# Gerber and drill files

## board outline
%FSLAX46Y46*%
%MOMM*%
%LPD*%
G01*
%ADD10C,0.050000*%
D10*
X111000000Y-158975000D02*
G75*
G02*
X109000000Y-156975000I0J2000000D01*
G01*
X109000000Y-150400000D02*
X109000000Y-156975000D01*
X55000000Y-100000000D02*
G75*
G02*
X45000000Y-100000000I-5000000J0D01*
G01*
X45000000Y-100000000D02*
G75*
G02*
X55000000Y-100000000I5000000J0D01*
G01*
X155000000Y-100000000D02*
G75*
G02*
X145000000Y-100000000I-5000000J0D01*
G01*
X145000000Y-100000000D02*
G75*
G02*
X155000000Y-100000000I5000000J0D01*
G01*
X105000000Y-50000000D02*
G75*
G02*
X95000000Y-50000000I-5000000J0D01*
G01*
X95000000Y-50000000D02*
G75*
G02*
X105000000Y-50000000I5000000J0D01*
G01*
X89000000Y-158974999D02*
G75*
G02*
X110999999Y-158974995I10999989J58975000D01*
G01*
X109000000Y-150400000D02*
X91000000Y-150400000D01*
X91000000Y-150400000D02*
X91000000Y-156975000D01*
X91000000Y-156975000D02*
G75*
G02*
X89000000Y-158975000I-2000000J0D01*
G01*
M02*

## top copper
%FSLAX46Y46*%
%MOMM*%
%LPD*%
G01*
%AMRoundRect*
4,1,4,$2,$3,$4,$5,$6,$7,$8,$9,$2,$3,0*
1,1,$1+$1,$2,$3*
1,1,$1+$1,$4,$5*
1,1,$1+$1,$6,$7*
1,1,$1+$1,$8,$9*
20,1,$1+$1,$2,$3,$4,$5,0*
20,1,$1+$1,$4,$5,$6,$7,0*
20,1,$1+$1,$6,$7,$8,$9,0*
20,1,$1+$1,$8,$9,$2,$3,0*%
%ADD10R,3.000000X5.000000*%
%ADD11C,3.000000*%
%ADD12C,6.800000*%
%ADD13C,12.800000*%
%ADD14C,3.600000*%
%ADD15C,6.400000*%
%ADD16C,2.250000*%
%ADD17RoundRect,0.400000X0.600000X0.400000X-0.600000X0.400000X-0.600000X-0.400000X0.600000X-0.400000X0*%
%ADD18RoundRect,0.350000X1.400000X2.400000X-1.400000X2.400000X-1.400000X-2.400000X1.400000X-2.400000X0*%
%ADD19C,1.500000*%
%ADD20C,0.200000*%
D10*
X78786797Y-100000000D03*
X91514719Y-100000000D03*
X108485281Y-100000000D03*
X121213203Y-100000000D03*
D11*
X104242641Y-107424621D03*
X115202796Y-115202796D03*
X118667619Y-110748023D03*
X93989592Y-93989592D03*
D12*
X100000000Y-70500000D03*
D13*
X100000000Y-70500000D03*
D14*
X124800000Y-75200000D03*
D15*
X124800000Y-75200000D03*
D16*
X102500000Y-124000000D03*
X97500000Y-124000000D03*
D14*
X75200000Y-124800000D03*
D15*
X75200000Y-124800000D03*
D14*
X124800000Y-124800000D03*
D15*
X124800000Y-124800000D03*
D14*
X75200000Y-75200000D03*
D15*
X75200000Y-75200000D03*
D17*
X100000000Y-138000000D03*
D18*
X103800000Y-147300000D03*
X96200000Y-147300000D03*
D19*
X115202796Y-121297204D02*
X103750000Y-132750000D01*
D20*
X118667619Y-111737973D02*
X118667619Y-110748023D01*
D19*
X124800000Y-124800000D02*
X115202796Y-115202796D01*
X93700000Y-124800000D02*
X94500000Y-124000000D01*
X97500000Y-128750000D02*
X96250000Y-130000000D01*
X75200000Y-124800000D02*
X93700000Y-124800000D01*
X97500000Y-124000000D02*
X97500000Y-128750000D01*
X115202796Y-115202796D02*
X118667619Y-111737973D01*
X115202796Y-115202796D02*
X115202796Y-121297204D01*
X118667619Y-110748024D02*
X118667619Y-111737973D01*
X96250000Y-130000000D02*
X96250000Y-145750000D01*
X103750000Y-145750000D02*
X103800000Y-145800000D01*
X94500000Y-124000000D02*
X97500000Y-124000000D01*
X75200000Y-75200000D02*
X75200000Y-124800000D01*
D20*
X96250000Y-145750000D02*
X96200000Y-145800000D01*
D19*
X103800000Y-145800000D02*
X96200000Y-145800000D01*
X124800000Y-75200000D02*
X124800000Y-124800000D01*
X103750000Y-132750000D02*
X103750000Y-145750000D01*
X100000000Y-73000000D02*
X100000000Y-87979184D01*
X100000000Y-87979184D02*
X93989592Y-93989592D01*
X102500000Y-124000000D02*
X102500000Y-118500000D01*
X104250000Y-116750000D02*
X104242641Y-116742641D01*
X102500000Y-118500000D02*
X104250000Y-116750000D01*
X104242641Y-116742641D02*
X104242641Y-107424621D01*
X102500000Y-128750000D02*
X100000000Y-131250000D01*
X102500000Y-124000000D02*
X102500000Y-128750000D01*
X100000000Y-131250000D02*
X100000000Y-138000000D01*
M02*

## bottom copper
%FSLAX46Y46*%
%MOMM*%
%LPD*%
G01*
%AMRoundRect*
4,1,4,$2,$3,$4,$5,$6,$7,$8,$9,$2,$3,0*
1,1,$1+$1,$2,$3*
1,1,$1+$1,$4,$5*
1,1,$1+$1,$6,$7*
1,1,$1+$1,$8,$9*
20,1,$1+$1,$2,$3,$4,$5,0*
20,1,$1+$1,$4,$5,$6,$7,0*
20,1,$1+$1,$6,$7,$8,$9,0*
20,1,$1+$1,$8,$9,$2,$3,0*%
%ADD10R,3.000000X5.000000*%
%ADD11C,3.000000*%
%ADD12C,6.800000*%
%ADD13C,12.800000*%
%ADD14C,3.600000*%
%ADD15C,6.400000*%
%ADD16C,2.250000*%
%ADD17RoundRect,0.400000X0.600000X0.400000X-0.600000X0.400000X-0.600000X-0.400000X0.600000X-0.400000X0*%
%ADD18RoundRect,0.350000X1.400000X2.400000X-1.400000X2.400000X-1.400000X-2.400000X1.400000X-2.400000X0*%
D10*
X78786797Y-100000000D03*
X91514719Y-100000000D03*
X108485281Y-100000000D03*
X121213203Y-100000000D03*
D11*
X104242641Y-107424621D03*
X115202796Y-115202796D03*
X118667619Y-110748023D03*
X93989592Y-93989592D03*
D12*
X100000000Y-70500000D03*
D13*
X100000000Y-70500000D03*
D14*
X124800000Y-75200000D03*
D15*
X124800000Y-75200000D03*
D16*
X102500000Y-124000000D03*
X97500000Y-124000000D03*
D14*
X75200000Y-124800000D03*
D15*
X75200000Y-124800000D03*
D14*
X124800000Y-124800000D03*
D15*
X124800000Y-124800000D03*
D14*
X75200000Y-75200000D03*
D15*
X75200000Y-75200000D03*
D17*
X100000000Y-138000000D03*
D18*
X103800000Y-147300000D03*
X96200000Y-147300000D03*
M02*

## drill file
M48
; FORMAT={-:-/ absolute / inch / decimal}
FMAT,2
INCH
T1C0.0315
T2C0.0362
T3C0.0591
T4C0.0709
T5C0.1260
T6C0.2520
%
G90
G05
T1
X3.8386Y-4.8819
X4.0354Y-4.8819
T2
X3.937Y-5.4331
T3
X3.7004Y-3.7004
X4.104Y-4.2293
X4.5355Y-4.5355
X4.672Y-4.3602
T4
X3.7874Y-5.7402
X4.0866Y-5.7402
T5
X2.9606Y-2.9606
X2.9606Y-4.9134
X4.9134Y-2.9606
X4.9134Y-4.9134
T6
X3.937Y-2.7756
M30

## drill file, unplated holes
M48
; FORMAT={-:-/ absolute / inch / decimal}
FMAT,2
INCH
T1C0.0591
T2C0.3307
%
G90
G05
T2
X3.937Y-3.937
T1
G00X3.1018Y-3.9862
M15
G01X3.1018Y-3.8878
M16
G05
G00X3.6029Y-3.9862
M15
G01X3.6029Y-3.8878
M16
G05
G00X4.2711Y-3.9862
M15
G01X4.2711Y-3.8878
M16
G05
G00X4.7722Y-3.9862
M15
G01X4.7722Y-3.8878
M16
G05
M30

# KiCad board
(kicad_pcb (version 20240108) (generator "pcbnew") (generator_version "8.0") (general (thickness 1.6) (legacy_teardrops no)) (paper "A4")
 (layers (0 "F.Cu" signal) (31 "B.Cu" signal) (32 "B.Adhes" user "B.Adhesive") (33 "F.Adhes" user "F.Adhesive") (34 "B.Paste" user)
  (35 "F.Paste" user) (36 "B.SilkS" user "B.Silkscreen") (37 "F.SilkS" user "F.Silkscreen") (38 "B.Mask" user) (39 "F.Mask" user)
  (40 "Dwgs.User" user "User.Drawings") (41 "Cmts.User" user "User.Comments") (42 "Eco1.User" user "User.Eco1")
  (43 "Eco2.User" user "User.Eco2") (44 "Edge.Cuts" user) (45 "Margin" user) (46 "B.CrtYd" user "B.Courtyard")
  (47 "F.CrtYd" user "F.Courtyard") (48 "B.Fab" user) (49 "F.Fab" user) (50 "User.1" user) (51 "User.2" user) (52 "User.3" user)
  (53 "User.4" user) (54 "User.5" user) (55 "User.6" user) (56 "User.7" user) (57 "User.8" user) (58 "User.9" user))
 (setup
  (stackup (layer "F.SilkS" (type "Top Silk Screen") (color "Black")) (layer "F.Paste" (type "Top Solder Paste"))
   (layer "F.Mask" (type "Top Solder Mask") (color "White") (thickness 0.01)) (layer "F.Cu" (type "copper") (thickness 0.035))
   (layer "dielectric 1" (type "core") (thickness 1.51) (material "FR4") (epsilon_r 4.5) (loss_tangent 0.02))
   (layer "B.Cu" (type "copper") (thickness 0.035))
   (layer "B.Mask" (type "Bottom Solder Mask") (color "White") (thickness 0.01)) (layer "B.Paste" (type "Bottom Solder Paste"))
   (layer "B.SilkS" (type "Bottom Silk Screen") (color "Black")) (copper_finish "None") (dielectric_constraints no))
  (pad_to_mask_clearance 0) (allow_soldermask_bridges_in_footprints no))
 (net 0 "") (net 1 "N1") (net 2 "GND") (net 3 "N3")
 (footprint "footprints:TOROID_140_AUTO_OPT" (layer "F.Cu") (at 100 100 45)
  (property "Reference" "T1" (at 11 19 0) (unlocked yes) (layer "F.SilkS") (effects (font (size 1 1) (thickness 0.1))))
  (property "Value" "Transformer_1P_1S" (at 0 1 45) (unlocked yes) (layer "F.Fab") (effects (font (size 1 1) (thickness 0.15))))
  (pad "" np_thru_hole rect (at -15 -15 90) (size 5 3) (drill oval 4 1.5) (layers "F&B.Cu"))
  (pad "" np_thru_hole rect (at -6 -6 90) (size 5 3) (drill oval 4 1.5) (layers "F&B.Cu"))
  (pad "" np_thru_hole rect (at 6 6 90) (size 5 3) (drill oval 4 1.5) (layers "F&B.Cu"))
  (pad "" np_thru_hole rect (at 15 15 90) (size 5 3) (drill oval 4 1.5) (layers "F&B.Cu"))
  (pad "1" thru_hole circle (at -2.25 8.25 45) (size 3 3) (drill 1.5) (layers "*.Cu" "*.Mask") (remove_unused_layers no) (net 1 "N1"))
  (pad "2" thru_hole circle (at 0 21.5 45) (size 3 3) (drill 1.5) (layers "*.Cu" "*.Mask") (remove_unused_layers no) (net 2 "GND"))
  (pad "3" thru_hole circle (at 5.6 20.8 45) (size 3 3) (drill 1.5) (layers "*.Cu" "*.Mask") (remove_unused_layers no) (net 2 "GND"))
  (pad "4" thru_hole circle (at 0 -8.500001 45) (size 3 3) (drill 1.5) (layers "*.Cu" "*.Mask") (remove_unused_layers no) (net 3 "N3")))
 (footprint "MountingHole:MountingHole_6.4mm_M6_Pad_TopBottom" (layer "F.Cu") (at 100 70.5)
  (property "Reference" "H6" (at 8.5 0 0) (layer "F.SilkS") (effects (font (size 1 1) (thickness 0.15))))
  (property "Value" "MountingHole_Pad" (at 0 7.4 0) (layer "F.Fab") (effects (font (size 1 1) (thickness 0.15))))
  (pad "1" thru_hole circle (at 0 0) (size 6.8 6.8) (drill 6.4) (layers "*.Cu" "*.Mask") (remove_unused_layers no) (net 3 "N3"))
  (pad "1" connect circle (at 0 0) (size 12.8 12.8) (layers "F.Cu" "F.Mask") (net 3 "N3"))
  (pad "1" connect circle (at 0 0) (size 12.8 12.8) (layers "B.Cu" "B.Mask") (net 3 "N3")))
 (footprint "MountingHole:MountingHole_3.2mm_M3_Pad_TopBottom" (layer "F.Cu") (at 124.8 75.2)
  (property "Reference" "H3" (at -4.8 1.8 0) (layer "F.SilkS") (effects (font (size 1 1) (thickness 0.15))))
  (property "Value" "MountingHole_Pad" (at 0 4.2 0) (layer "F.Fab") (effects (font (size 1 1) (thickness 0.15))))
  (pad "1" thru_hole circle (at 0 0) (size 3.6 3.6) (drill 3.2) (layers "*.Cu" "*.Mask") (remove_unused_layers no) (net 2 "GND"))
  (pad "1" connect circle (at 0 0) (size 6.4 6.4) (layers "F.Cu" "F.Mask") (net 2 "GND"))
  (pad "1" connect circle (at 0 0) (size 6.4 6.4) (layers "B.Cu" "B.Mask") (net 2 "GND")))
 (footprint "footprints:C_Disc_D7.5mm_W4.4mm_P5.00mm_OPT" (layer "F.Cu") (at 102.5 124 180)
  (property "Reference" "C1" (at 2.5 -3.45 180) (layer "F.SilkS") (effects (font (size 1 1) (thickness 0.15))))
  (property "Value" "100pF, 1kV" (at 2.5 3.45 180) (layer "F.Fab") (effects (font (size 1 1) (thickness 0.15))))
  (pad "1" thru_hole circle (at 0 0 180) (size 2.25 2.25) (drill 0.8) (layers "*.Cu" "*.Mask") (remove_unused_layers no) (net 1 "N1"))
  (pad "2" thru_hole circle (at 5 0 180) (size 2.25 2.25) (drill 0.8) (layers "*.Cu" "*.Mask") (remove_unused_layers no) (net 2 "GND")))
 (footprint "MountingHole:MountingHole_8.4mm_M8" (layer "F.Cu") (at 100 100)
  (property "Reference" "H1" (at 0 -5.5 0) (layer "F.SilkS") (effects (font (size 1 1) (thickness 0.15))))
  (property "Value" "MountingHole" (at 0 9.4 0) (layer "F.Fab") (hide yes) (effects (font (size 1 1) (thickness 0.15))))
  (pad "" np_thru_hole circle (at 0 0) (size 8.4 8.4) (drill 8.4) (layers "*.Cu" "*.Mask")))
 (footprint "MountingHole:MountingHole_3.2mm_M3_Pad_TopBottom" (layer "F.Cu") (at 75.2 124.8)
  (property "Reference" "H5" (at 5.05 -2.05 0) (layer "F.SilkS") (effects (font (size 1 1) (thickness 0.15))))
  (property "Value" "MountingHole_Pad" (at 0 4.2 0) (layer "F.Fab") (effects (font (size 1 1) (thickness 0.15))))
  (pad "1" thru_hole circle (at 0 0) (size 3.6 3.6) (drill 3.2) (layers "*.Cu" "*.Mask") (remove_unused_layers no) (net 2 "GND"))
  (pad "1" connect circle (at 0 0) (size 6.4 6.4) (layers "F.Cu" "F.Mask") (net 2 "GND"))
  (pad "1" connect circle (at 0 0) (size 6.4 6.4) (layers "B.Cu" "B.Mask") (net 2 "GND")))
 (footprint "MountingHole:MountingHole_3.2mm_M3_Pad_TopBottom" (layer "F.Cu") (at 124.8 124.8)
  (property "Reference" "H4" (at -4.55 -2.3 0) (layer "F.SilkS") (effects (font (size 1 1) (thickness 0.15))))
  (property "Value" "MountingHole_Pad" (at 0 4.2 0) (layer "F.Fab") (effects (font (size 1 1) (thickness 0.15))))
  (pad "1" thru_hole circle (at 0 0) (size 3.6 3.6) (drill 3.2) (layers "*.Cu" "*.Mask") (remove_unused_layers no) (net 2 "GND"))
  (pad "1" connect circle (at 0 0) (size 6.4 6.4) (layers "F.Cu" "F.Mask") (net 2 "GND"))
  (pad "1" connect circle (at 0 0) (size 6.4 6.4) (layers "B.Cu" "B.Mask") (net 2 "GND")))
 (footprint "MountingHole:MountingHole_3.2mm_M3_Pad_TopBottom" (layer "F.Cu") (at 75.2 75.2)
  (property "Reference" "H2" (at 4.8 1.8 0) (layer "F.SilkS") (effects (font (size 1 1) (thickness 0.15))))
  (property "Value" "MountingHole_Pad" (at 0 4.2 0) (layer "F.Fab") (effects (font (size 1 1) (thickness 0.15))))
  (pad "1" thru_hole circle (at 0 0) (size 3.6 3.6) (drill 3.2) (layers "*.Cu" "*.Mask") (remove_unused_layers no) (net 2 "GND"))
  (pad "1" connect circle (at 0 0) (size 6.4 6.4) (layers "F.Cu" "F.Mask") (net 2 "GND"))
  (pad "1" connect circle (at 0 0) (size 6.4 6.4) (layers "B.Cu" "B.Mask") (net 2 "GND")))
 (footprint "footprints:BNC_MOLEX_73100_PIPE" (layer "F.Cu") (at 100 138 180)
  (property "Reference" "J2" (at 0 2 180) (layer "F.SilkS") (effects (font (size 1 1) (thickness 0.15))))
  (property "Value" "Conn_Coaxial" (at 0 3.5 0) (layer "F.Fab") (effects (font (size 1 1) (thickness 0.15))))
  (pad "1" thru_hole roundrect (at 0 0 180) (size 2 1.6) (drill 0.92) (layers "*.Cu" "*.Mask") (remove_unused_layers no)
   (roundrect_rratio 0.25) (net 1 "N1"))
  (pad "2" thru_hole roundrect (at -3.8 -7.8 180) (size 3.5 5.5) (drill 1.8 (offset 0 -1.5)) (layers "*.Cu" "*.Mask")
   (remove_unused_layers no) (roundrect_rratio 0.1) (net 2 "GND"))
  (pad "2" thru_hole roundrect (at 3.8 -7.8 180) (size 3.5 5.5) (drill 1.8 (offset 0 -1.5)) (layers "*.Cu" "*.Mask")
   (remove_unused_layers no) (roundrect_rratio 0.1) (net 2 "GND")))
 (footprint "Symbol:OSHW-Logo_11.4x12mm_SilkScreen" (layer "B.Cu") (at 65 110.5 180)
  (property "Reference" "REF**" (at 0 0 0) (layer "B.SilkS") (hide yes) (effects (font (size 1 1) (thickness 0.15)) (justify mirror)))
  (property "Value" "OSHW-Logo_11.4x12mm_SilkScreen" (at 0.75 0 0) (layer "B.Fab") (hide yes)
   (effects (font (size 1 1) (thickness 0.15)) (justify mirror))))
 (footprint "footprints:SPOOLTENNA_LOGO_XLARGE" (layer "B.Cu") (at 100 60 180)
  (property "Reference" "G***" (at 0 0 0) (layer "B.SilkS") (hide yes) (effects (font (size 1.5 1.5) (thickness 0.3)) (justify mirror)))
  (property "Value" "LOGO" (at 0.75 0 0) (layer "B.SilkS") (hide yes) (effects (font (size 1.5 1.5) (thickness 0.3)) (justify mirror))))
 (gr_arc (start 111 158.975) (mid 109.585786 158.389214) (end 109 156.975) (stroke (width 0.05) (type default)) (layer "Edge.Cuts"))
 (gr_line (start 109 150.4) (end 109 156.975) (stroke (width 0.05) (type default)) (layer "Edge.Cuts"))
 (gr_circle (center 50 100) (end 55 100) (stroke (width 0.05) (type default)) (fill none) (layer "Edge.Cuts"))
 (gr_circle (center 150 100) (end 155 100) (stroke (width 0.05) (type default)) (fill none) (layer "Edge.Cuts"))
 (gr_circle (center 100 50) (end 105 50) (stroke (width 0.05) (type default)) (fill none) (layer "Edge.Cuts"))
 (gr_arc (start 89 158.974999) (mid 99.999974 40.007913) (end 110.999999 158.974995) (stroke (width 0.05) (type default))
  (layer "Edge.Cuts"))
 (gr_line (start 109 150.4) (end 91 150.4) (stroke (width 0.05) (type default)) (layer "Edge.Cuts"))
 (gr_line (start 91 150.4) (end 91 156.975) (stroke (width 0.05) (type default)) (layer "Edge.Cuts"))
 (gr_arc (start 91 156.975) (mid 90.414214 158.389214) (end 89 158.975) (stroke (width 0.05) (type default)) (layer "Edge.Cuts"))
 (segment (start 115.202796 121.297204) (end 103.75 132.75) (width 1.5) (layer "F.Cu") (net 2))
 (segment (start 118.667619 111.737973) (end 118.667619 110.748023) (width 0.2) (layer "F.Cu") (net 2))
 (segment (start 124.8 124.8) (end 115.202796 115.202796) (width 1.5) (layer "F.Cu") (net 2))
 (segment (start 93.7 124.8) (end 94.5 124) (width 1.5) (layer "F.Cu") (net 2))
 (segment (start 97.5 128.75) (end 96.25 130) (width 1.5) (layer "F.Cu") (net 2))
 (segment (start 75.2 124.8) (end 93.7 124.8) (width 1.5) (layer "F.Cu") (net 2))
 (segment (start 97.5 124) (end 97.5 128.75) (width 1.5) (layer "F.Cu") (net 2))
 (segment (start 115.202796 115.202796) (end 118.667619 111.737973) (width 1.5) (layer "F.Cu") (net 2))
 (segment (start 115.202796 115.202796) (end 115.202796 121.297204) (width 1.5) (layer "F.Cu") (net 2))
 (segment (start 118.667619 110.748024) (end 118.667619 111.737973) (width 1.5) (layer "F.Cu") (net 2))
 (segment (start 96.25 130) (end 96.25 145.75) (width 1.5) (layer "F.Cu") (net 2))
 (segment (start 103.75 145.75) (end 103.8 145.8) (width 1.5) (layer "F.Cu") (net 2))
 (segment (start 94.5 124) (end 97.5 124) (width 1.5) (layer "F.Cu") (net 2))
 (segment (start 75.2 75.2) (end 75.2 124.8) (width 1.5) (layer "F.Cu") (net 2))
 (segment (start 96.25 145.75) (end 96.2 145.8) (width 0.2) (layer "F.Cu") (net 2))
 (segment (start 103.8 145.8) (end 96.2 145.8) (width 1.5) (layer "F.Cu") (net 2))
 (segment (start 124.8 75.2) (end 124.8 124.8) (width 1.5) (layer "F.Cu") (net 2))
 (segment (start 103.75 132.75) (end 103.75 145.75) (width 1.5) (layer "F.Cu") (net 2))
 (segment (start 100 73) (end 100 87.979184) (width 1.5) (layer "F.Cu") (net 3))
 (segment (start 100 87.979184) (end 93.989592 93.989592) (width 1.5) (layer "F.Cu") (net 3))
 (segment (start 102.5 124) (end 102.5 118.5) (width 1.5) (layer "F.Cu") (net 1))
 (segment (start 104.25 116.75) (end 104.242641 116.742641) (width 1.5) (layer "F.Cu") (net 1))
 (segment (start 102.5 118.5) (end 104.25 116.75) (width 1.5) (layer "F.Cu") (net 1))
 (segment (start 104.242641 116.742641) (end 104.242641 107.424621) (width 1.5) (layer "F.Cu") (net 1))
 (segment (start 102.5 128.75) (end 100 131.25) (width 1.5) (layer "F.Cu") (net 1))
 (segment (start 102.5 124) (end 102.5 128.75) (width 1.5) (layer "F.Cu") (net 1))
 (segment (start 100 131.25) (end 100 138) (width 1.5) (layer "F.Cu") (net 1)))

